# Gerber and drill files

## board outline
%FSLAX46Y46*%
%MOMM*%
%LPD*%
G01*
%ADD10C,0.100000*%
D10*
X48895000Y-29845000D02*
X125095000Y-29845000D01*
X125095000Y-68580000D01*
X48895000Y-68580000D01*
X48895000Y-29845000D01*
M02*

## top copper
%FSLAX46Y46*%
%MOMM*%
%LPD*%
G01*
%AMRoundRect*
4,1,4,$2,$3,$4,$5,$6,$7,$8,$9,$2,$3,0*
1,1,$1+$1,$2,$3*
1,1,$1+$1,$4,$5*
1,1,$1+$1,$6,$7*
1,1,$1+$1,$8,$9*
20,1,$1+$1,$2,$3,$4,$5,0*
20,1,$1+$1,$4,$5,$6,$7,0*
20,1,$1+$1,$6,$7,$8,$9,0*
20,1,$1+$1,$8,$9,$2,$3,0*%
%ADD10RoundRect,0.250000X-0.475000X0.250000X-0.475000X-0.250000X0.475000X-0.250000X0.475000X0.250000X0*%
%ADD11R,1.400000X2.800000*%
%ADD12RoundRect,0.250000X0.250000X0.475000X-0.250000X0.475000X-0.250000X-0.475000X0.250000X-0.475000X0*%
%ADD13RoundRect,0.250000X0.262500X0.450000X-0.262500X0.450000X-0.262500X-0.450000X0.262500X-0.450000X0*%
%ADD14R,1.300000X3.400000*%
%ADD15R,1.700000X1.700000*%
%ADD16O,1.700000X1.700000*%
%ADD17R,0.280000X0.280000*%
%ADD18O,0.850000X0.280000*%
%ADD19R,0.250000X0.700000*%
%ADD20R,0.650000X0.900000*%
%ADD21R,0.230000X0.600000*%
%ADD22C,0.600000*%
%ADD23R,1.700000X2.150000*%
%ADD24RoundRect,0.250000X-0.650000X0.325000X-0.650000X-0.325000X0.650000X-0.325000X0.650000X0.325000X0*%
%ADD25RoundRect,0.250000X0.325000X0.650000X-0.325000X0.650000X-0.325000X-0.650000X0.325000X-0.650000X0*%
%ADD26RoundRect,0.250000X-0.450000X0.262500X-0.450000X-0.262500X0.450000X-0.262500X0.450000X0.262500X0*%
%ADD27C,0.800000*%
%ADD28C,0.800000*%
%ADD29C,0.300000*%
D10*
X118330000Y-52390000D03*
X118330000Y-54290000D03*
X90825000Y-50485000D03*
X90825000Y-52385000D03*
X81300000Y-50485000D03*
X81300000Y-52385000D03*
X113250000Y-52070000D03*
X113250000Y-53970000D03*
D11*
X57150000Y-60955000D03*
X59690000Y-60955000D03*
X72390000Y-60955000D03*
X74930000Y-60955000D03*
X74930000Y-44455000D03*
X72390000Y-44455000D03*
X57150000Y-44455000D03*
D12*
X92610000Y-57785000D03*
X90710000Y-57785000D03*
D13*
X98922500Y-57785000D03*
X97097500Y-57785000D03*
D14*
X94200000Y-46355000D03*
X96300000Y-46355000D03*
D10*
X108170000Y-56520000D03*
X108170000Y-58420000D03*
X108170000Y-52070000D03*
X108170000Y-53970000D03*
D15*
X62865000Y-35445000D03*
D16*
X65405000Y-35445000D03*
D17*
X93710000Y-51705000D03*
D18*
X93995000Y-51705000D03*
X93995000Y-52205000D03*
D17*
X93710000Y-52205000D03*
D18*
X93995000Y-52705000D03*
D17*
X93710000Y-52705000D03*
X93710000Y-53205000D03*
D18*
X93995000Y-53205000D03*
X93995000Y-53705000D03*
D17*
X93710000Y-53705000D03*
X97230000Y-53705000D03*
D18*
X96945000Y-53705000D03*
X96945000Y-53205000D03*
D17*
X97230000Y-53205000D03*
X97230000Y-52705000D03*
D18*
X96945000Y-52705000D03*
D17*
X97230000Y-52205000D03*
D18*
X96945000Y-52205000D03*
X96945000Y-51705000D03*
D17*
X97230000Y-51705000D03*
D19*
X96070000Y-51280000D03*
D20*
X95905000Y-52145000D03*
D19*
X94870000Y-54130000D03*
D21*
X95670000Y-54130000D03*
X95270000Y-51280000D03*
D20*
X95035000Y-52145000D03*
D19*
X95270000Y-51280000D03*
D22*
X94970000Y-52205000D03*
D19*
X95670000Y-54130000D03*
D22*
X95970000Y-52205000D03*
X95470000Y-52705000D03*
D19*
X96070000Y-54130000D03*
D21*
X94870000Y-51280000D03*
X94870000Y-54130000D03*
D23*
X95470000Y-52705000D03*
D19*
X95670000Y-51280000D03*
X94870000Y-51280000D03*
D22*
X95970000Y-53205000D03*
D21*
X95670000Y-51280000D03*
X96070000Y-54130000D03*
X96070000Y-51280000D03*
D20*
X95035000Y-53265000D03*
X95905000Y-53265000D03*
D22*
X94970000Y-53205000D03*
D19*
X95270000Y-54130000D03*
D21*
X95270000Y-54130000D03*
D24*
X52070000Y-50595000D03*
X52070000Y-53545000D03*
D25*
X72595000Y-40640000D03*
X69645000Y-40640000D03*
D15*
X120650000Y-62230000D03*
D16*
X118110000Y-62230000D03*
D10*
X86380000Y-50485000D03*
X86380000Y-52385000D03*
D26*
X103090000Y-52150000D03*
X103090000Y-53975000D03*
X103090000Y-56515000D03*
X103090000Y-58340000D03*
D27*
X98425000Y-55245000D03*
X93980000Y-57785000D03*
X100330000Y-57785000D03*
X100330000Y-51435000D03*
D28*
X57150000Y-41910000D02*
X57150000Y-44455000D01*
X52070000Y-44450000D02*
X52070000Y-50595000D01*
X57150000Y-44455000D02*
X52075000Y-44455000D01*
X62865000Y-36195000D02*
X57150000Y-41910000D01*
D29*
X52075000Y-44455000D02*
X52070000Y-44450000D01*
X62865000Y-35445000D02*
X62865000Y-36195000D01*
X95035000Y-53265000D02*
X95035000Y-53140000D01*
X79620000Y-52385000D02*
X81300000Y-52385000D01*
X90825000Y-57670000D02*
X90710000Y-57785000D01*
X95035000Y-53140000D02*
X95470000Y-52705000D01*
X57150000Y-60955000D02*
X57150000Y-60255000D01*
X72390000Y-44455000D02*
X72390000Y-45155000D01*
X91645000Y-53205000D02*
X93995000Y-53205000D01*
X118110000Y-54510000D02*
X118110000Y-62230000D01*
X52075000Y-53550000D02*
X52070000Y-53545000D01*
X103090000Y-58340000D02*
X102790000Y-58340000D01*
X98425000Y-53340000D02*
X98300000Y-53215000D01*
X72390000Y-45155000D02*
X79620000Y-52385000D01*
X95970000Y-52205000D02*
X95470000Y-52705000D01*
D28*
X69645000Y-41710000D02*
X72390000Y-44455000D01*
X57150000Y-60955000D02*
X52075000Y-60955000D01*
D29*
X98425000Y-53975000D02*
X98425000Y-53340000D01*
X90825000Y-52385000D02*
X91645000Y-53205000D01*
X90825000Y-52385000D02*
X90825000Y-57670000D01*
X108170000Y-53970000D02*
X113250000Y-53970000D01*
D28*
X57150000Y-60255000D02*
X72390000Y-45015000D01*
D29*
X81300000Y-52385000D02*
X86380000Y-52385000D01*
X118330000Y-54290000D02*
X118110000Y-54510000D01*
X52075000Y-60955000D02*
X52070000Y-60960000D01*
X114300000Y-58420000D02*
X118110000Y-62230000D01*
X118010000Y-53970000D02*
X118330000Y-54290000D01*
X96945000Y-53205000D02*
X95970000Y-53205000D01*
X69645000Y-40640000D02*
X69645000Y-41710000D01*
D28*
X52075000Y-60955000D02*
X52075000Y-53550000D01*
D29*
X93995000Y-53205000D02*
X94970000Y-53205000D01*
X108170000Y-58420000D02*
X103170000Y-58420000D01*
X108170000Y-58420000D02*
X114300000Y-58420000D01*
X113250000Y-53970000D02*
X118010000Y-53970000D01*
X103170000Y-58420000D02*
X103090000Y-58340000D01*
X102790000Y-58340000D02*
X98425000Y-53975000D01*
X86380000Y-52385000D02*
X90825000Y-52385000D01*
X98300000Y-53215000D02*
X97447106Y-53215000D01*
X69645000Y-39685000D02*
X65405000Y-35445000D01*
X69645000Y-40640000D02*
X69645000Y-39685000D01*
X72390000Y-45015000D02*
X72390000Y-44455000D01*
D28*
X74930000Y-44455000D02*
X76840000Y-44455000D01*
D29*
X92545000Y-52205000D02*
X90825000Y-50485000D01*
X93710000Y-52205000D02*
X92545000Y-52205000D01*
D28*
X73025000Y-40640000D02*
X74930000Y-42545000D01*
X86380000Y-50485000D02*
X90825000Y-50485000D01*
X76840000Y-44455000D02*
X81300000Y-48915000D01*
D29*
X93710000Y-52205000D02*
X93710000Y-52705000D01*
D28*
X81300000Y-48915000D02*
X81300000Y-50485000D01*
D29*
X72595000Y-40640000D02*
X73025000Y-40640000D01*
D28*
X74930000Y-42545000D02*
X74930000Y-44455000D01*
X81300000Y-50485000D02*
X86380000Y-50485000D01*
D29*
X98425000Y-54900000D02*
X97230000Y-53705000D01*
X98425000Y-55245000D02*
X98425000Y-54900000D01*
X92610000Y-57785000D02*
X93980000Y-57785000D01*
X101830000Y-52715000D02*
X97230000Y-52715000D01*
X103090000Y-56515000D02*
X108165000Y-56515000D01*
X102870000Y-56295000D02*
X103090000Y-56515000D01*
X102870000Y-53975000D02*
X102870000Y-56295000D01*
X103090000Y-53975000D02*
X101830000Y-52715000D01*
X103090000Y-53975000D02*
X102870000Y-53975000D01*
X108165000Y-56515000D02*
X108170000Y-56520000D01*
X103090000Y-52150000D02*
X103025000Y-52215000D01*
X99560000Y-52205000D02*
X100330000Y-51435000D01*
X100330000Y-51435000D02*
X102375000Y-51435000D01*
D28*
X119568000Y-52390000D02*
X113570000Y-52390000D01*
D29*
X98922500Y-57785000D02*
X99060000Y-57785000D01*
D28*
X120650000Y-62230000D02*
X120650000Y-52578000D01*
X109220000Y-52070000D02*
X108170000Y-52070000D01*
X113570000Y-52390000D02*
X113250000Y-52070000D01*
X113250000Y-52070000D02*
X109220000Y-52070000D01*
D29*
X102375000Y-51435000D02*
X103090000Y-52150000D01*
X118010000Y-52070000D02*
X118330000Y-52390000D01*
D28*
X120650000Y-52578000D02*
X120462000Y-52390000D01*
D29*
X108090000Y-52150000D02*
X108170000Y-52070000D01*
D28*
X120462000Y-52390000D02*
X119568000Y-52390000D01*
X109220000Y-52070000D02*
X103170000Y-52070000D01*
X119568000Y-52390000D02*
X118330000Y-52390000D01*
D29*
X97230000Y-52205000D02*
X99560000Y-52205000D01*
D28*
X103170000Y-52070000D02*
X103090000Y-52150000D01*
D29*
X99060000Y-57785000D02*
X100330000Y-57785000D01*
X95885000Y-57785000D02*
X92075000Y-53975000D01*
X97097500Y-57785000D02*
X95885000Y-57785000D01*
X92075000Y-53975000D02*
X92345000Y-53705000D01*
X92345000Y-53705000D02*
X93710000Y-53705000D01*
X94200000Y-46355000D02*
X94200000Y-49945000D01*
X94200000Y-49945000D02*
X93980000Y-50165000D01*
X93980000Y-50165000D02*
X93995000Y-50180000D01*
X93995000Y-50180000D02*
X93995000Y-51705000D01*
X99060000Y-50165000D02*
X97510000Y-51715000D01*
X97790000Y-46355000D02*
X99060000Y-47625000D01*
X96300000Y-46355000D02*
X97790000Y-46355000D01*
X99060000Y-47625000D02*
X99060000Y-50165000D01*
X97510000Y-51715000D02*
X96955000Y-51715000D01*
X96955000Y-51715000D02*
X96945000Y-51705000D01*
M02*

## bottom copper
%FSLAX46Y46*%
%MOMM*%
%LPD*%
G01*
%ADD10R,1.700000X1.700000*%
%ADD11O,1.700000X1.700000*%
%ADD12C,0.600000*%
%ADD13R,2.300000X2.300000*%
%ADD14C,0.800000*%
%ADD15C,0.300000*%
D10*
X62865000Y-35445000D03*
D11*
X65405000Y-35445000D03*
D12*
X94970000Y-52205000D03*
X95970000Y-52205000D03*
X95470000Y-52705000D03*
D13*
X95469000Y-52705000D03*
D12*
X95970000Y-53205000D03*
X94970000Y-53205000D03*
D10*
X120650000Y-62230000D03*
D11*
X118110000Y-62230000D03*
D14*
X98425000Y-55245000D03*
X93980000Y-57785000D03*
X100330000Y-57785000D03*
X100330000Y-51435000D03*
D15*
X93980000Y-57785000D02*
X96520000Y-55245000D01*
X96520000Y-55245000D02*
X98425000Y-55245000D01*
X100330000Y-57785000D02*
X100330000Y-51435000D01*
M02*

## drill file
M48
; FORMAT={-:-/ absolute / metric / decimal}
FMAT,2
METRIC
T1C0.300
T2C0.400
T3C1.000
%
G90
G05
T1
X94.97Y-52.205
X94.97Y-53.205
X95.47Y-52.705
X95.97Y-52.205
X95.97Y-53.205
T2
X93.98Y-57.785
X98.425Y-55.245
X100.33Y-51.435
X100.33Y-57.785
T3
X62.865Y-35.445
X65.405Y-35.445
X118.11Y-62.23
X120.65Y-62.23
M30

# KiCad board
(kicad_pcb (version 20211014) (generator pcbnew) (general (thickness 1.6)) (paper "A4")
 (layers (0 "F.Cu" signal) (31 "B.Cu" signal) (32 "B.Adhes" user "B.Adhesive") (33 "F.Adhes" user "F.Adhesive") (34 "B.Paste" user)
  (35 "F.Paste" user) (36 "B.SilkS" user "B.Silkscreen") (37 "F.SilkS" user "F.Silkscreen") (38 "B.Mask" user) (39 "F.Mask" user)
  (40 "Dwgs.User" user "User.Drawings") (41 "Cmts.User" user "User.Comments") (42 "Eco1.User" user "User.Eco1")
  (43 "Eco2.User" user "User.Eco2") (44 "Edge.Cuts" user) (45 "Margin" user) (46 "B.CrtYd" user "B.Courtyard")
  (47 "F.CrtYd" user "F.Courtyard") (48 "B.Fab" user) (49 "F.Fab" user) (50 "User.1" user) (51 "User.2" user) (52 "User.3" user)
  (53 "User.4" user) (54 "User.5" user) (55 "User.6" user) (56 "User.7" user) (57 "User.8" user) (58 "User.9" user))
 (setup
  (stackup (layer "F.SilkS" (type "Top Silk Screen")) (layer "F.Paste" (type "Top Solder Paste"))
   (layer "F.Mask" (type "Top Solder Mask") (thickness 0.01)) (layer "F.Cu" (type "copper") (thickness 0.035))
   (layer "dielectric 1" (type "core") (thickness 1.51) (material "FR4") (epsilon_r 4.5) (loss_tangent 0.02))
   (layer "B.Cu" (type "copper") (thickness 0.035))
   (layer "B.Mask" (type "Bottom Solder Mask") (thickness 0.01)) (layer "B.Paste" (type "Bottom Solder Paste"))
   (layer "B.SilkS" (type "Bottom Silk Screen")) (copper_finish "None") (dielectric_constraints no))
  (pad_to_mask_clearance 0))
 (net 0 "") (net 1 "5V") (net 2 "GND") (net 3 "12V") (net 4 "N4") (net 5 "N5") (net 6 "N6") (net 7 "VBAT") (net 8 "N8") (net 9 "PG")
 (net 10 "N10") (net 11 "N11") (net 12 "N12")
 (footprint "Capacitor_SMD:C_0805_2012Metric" (layer "F.Cu") (at 118.33 53.34 -90)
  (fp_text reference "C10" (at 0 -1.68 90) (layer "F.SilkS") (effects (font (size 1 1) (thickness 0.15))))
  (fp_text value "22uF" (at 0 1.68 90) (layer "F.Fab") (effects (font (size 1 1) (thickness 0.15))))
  (pad "1" smd roundrect (at -0.95 0 270) (size 1 1.45) (layers "F.Cu" "F.Paste" "F.Mask") (roundrect_rratio 0.25) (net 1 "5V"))
  (pad "2" smd roundrect (at 0.95 0 270) (size 1 1.45) (layers "F.Cu" "F.Paste" "F.Mask") (roundrect_rratio 0.25) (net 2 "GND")))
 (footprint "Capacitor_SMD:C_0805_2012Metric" (layer "F.Cu") (at 90.825 51.435 -90)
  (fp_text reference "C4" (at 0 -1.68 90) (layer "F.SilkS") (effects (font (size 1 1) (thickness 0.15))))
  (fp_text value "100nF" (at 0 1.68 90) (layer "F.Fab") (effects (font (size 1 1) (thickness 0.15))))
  (pad "1" smd roundrect (at -0.95 0 270) (size 1 1.45) (layers "F.Cu" "F.Paste" "F.Mask") (roundrect_rratio 0.25) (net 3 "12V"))
  (pad "2" smd roundrect (at 0.95 0 270) (size 1 1.45) (layers "F.Cu" "F.Paste" "F.Mask") (roundrect_rratio 0.25) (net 2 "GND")))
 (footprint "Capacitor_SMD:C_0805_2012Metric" (layer "F.Cu") (at 81.3 51.435 -90)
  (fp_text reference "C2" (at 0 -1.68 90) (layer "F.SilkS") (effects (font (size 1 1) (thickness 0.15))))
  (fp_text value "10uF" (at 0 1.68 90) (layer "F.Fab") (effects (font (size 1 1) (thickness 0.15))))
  (pad "1" smd roundrect (at -0.95 0 270) (size 1 1.45) (layers "F.Cu" "F.Paste" "F.Mask") (roundrect_rratio 0.25) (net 3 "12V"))
  (pad "2" smd roundrect (at 0.95 0 270) (size 1 1.45) (layers "F.Cu" "F.Paste" "F.Mask") (roundrect_rratio 0.25) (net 2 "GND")))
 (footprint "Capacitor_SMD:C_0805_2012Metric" (layer "F.Cu") (at 113.25 53.02 -90)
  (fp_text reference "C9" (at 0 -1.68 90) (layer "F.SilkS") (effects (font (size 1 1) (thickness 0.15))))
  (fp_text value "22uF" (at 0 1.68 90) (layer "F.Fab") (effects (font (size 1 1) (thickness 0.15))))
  (pad "1" smd roundrect (at -0.95 0 270) (size 1 1.45) (layers "F.Cu" "F.Paste" "F.Mask") (roundrect_rratio 0.25) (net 1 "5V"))
  (pad "2" smd roundrect (at 0.95 0 270) (size 1 1.45) (layers "F.Cu" "F.Paste" "F.Mask") (roundrect_rratio 0.25) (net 2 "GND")))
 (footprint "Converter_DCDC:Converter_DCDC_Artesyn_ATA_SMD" (layer "F.Cu") (at 66.04 52.705 90)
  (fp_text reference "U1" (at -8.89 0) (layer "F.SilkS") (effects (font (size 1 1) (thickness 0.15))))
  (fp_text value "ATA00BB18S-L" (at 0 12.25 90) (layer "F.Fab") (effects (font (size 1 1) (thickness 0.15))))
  (pad "1" smd rect (at -8.25 -8.89 90) (size 2.8 1.4) (layers "F.Cu" "F.Paste" "F.Mask") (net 2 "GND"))
  (pad "2" smd rect (at -8.25 -6.35 90) (size 2.8 1.4) (layers "F.Cu" "F.Paste" "F.Mask") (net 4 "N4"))
  (pad "7" smd rect (at -8.25 6.35 90) (size 2.8 1.4) (layers "F.Cu" "F.Paste" "F.Mask") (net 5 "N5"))
  (pad "8" smd rect (at -8.25 8.89 90) (size 2.8 1.4) (layers "F.Cu" "F.Paste" "F.Mask") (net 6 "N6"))
  (pad "9" smd rect (at 8.25 8.89 90) (size 2.8 1.4) (layers "F.Cu" "F.Paste" "F.Mask") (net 3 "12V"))
  (pad "10" smd rect (at 8.25 6.35 90) (size 2.8 1.4) (layers "F.Cu" "F.Paste" "F.Mask") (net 2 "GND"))
  (pad "16" smd rect (at 8.25 -8.89 90) (size 2.8 1.4) (layers "F.Cu" "F.Paste" "F.Mask") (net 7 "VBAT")))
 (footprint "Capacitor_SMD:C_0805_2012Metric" (layer "F.Cu") (at 91.66 57.785 180)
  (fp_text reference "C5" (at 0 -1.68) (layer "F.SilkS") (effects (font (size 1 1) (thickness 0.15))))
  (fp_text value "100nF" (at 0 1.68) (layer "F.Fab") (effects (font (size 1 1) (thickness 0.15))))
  (pad "1" smd roundrect (at -0.95 0 180) (size 1 1.45) (layers "F.Cu" "F.Paste" "F.Mask") (roundrect_rratio 0.25) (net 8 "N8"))
  (pad "2" smd roundrect (at 0.95 0 180) (size 1 1.45) (layers "F.Cu" "F.Paste" "F.Mask") (roundrect_rratio 0.25) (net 2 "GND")))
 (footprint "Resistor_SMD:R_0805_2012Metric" (layer "F.Cu") (at 98.01 57.785 180)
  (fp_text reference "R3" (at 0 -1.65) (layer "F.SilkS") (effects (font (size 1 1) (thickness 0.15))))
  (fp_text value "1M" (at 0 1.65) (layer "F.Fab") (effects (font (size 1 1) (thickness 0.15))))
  (pad "1" smd roundrect (at -0.9125 0 180) (size 1.025 1.4) (layers "F.Cu" "F.Paste" "F.Mask") (roundrect_rratio 0.243902439) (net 1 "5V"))
  (pad "2" smd roundrect (at 0.9125 0 180) (size 1.025 1.4) (layers "F.Cu" "F.Paste" "F.Mask") (roundrect_rratio 0.243902439) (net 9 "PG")))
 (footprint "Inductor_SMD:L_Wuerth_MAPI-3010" (layer "F.Cu") (at 95.25 46.355)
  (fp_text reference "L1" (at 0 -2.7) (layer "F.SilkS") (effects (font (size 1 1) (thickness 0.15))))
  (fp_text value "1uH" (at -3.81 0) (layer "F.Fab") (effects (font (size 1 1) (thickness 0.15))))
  (pad "1" smd rect (at -1.05 0) (size 1.3 3.4) (layers "F.Cu" "F.Paste" "F.Mask") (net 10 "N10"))
  (pad "2" smd rect (at 1.05 0) (size 1.3 3.4) (layers "F.Cu" "F.Paste" "F.Mask") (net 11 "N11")))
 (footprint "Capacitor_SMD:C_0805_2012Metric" (layer "F.Cu") (at 108.17 57.47 -90)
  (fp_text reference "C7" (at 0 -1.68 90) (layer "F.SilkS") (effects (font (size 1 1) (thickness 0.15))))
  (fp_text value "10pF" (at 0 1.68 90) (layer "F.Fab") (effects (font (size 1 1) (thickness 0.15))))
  (pad "1" smd roundrect (at -0.95 0 270) (size 1 1.45) (layers "F.Cu" "F.Paste" "F.Mask") (roundrect_rratio 0.25) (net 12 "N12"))
  (pad "2" smd roundrect (at 0.95 0 270) (size 1 1.45) (layers "F.Cu" "F.Paste" "F.Mask") (roundrect_rratio 0.25) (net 2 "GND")))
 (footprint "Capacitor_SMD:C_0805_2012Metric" (layer "F.Cu") (at 108.17 53.02 -90)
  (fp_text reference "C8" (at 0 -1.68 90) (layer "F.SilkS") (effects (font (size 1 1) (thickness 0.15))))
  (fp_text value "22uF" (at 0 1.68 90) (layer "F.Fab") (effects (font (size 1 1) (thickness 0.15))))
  (pad "1" smd roundrect (at -0.95 0 270) (size 1 1.45) (layers "F.Cu" "F.Paste" "F.Mask") (roundrect_rratio 0.25) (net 1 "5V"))
  (pad "2" smd roundrect (at 0.95 0 270) (size 1 1.45) (layers "F.Cu" "F.Paste" "F.Mask") (roundrect_rratio 0.25) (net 2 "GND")))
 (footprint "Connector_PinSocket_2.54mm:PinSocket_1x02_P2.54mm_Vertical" (layer "F.Cu") (at 62.865 35.445 90)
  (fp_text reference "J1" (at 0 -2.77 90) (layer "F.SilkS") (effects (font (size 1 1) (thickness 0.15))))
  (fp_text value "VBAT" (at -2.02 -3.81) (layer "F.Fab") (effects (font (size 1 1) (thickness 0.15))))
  (pad "1" thru_hole rect (at 0 0 90) (size 1.7 1.7) (drill 1) (layers *.Cu *.Mask) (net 7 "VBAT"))
  (pad "2" thru_hole oval (at 0 2.54 90) (size 1.7 1.7) (drill 1) (layers *.Cu *.Mask) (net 2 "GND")))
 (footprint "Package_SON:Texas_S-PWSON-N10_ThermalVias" (layer "F.Cu") (at 95.47 52.705)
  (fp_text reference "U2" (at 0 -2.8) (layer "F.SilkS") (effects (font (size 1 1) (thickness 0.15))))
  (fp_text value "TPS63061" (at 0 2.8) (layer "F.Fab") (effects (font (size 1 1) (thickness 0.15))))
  (pad "1" smd rect (at -1.76 -1) (size 0.28 0.28) (layers "F.Cu" "F.Paste" "F.Mask") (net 10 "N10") (solder_mask_margin 0.07)
   (solder_paste_margin -0.025))
  (pad "1" smd oval (at -1.475 -1) (size 0.85 0.28) (layers "F.Cu" "F.Paste" "F.Mask") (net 10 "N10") (solder_mask_margin 0.07)
   (solder_paste_margin -0.025))
  (pad "2" smd oval (at -1.475 -0.5) (size 0.85 0.28) (layers "F.Cu" "F.Paste" "F.Mask") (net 3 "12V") (solder_mask_margin 0.07)
   (solder_paste_margin -0.025))
  (pad "2" smd rect (at -1.76 -0.5) (size 0.28 0.28) (layers "F.Cu" "F.Paste" "F.Mask") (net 3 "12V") (solder_mask_margin 0.07)
   (solder_paste_margin -0.025))
  (pad "3" smd oval (at -1.475 0) (size 0.85 0.28) (layers "F.Cu" "F.Paste" "F.Mask") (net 3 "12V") (solder_mask_margin 0.07)
   (solder_paste_margin -0.025))
  (pad "3" smd rect (at -1.76 0) (size 0.28 0.28) (layers "F.Cu" "F.Paste" "F.Mask") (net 3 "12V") (solder_mask_margin 0.07)
   (solder_paste_margin -0.025))
  (pad "4" smd rect (at -1.76 0.5) (size 0.28 0.28) (layers "F.Cu" "F.Paste" "F.Mask") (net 2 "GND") (solder_mask_margin 0.07)
   (solder_paste_margin -0.025))
  (pad "4" smd oval (at -1.475 0.5) (size 0.85 0.28) (layers "F.Cu" "F.Paste" "F.Mask") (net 2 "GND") (solder_mask_margin 0.07)
   (solder_paste_margin -0.025))
  (pad "5" smd oval (at -1.475 1) (size 0.85 0.28) (layers "F.Cu" "F.Paste" "F.Mask") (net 9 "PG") (solder_mask_margin 0.07)
   (solder_paste_margin -0.025))
  (pad "5" smd rect (at -1.76 1) (size 0.28 0.28) (layers "F.Cu" "F.Paste" "F.Mask") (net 9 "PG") (solder_mask_margin 0.07)
   (solder_paste_margin -0.025))
  (pad "6" smd rect (at 1.76 1) (size 0.28 0.28) (layers "F.Cu" "F.Paste" "F.Mask") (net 8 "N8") (solder_mask_margin 0.07)
   (solder_paste_margin -0.025))
  (pad "6" smd oval (at 1.475 1) (size 0.85 0.28) (layers "F.Cu" "F.Paste" "F.Mask") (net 8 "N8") (solder_mask_margin 0.07)
   (solder_paste_margin -0.025))
  (pad "7" smd oval (at 1.475 0.5) (size 0.85 0.28) (layers "F.Cu" "F.Paste" "F.Mask") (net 2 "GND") (solder_mask_margin 0.07)
   (solder_paste_margin -0.025))
  (pad "7" smd rect (at 1.76 0.5) (size 0.28 0.28) (layers "F.Cu" "F.Paste" "F.Mask") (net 2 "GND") (solder_mask_margin 0.07)
   (solder_paste_margin -0.025))
  (pad "8" smd rect (at 1.76 0) (size 0.28 0.28) (layers "F.Cu" "F.Paste" "F.Mask") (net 12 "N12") (solder_mask_margin 0.07)
   (solder_paste_margin -0.025))
  (pad "8" smd oval (at 1.475 0) (size 0.85 0.28) (layers "F.Cu" "F.Paste" "F.Mask") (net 12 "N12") (solder_mask_margin 0.07)
   (solder_paste_margin -0.025))
  (pad "9" smd rect (at 1.76 -0.5) (size 0.28 0.28) (layers "F.Cu" "F.Paste" "F.Mask") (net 1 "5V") (solder_mask_margin 0.07)
   (solder_paste_margin -0.025))
  (pad "9" smd oval (at 1.475 -0.5) (size 0.85 0.28) (layers "F.Cu" "F.Paste" "F.Mask") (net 1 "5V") (solder_mask_margin 0.07)
   (solder_paste_margin -0.025))
  (pad "10" smd oval (at 1.475 -1) (size 0.85 0.28) (layers "F.Cu" "F.Paste" "F.Mask") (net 11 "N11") (solder_mask_margin 0.07)
   (solder_paste_margin -0.025))
  (pad "10" smd rect (at 1.76 -1) (size 0.28 0.28) (layers "F.Cu" "F.Paste" "F.Mask") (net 11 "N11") (solder_mask_margin 0.07)
   (solder_paste_margin -0.025))
  (pad "11" smd rect (at 0.6 -1.425) (size 0.25 0.7) (layers "F.Cu" "F.Paste" "F.Mask") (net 2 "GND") (solder_paste_margin -0.05))
  (pad "11" smd rect (at 0.435 -0.56) (size 0.65 0.9) (layers "F.Cu" "F.Paste" "F.Mask") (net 2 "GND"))
  (pad "11" smd rect (at -0.6 1.425) (size 0.25 0.7) (layers "F.Cu" "F.Paste" "F.Mask") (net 2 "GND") (solder_paste_margin -0.05))
  (pad "11" smd rect (at 0.2 1.425) (size 0.23 0.6) (layers "F.Cu" "F.Paste" "F.Mask") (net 2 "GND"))
  (pad "11" smd rect (at -0.2 -1.425) (size 0.23 0.6) (layers "F.Cu" "F.Paste" "F.Mask") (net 2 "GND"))
  (pad "11" smd rect (at -0.435 -0.56) (size 0.65 0.9) (layers "F.Cu" "F.Paste" "F.Mask") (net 2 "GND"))
  (pad "11" smd rect (at -0.2 -1.425) (size 0.25 0.7) (layers "F.Cu" "F.Paste" "F.Mask") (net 2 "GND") (solder_paste_margin -0.05))
  (pad "11" thru_hole circle (at -0.5 -0.5) (size 0.6 0.6) (drill 0.3) (layers *.Cu *.Mask) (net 2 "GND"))
  (pad "11" smd rect (at 0.2 1.425) (size 0.25 0.7) (layers "F.Cu" "F.Paste" "F.Mask") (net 2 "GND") (solder_paste_margin -0.05))
  (pad "11" thru_hole circle (at 0.5 -0.5) (size 0.6 0.6) (drill 0.3) (layers *.Cu *.Mask) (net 2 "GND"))
  (pad "11" thru_hole circle (at 0 0) (size 0.6 0.6) (drill 0.3) (layers *.Cu *.Mask) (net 2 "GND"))
  (pad "11" smd rect (at 0.6 1.425) (size 0.25 0.7) (layers "F.Cu" "F.Paste" "F.Mask") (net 2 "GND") (solder_paste_margin -0.05))
  (pad "11" smd rect (at -0.6 -1.425) (size 0.23 0.6) (layers "F.Cu" "F.Paste" "F.Mask") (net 2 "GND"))
  (pad "11" smd rect (at -0.6 1.425) (size 0.23 0.6) (layers "F.Cu" "F.Paste" "F.Mask") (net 2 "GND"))
  (pad "11" smd rect (at 0 0) (size 1.7 2.15) (layers "F.Cu" "F.Mask") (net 2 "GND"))
  (pad "11" smd rect (at -0.001 0) (size 2.3 2.3) (layers "B.Cu") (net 2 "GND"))
  (pad "11" smd rect (at 0.2 -1.425) (size 0.25 0.7) (layers "F.Cu" "F.Paste" "F.Mask") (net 2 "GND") (solder_paste_margin -0.05))
  (pad "11" smd rect (at -0.6 -1.425) (size 0.25 0.7) (layers "F.Cu" "F.Paste" "F.Mask") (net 2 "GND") (solder_paste_margin -0.05))
  (pad "11" thru_hole circle (at 0.5 0.5) (size 0.6 0.6) (drill 0.3) (layers *.Cu *.Mask) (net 2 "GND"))
  (pad "11" smd rect (at 0.2 -1.425) (size 0.23 0.6) (layers "F.Cu" "F.Paste" "F.Mask") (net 2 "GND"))
  (pad "11" smd rect (at 0.6 1.425) (size 0.23 0.6) (layers "F.Cu" "F.Paste" "F.Mask") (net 2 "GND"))
  (pad "11" smd rect (at 0.6 -1.425) (size 0.23 0.6) (layers "F.Cu" "F.Paste" "F.Mask") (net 2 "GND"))
  (pad "11" smd rect (at -0.435 0.56) (size 0.65 0.9) (layers "F.Cu" "F.Paste" "F.Mask") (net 2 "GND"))
  (pad "11" smd rect (at 0.435 0.56) (size 0.65 0.9) (layers "F.Cu" "F.Paste" "F.Mask") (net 2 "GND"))
  (pad "11" thru_hole circle (at -0.5 0.5) (size 0.6 0.6) (drill 0.3) (layers *.Cu *.Mask) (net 2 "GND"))
  (pad "11" smd rect (at -0.2 1.425) (size 0.25 0.7) (layers "F.Cu" "F.Paste" "F.Mask") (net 2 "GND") (solder_paste_margin -0.05))
  (pad "11" smd rect (at -0.2 1.425) (size 0.23 0.6) (layers "F.Cu" "F.Paste" "F.Mask") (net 2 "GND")))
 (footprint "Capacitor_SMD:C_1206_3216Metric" (layer "F.Cu") (at 52.07 52.07 -90)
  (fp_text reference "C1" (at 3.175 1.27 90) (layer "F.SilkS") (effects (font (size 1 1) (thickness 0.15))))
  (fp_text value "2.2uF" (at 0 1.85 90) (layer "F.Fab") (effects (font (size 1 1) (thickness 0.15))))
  (pad "1" smd roundrect (at -1.475 0 270) (size 1.15 1.8) (layers "F.Cu" "F.Paste" "F.Mask") (roundrect_rratio 0.2173913043) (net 7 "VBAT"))
  (pad "2" smd roundrect (at 1.475 0 270) (size 1.15 1.8) (layers "F.Cu" "F.Paste" "F.Mask") (roundrect_rratio 0.2173913043) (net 2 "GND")))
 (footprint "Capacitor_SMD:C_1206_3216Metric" (layer "F.Cu") (at 71.12 40.64 180)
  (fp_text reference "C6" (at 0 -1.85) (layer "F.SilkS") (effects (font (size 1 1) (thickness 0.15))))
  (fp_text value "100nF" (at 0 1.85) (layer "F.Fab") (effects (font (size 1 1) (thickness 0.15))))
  (pad "1" smd roundrect (at -1.475 0 180) (size 1.15 1.8) (layers "F.Cu" "F.Paste" "F.Mask") (roundrect_rratio 0.2173913043) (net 3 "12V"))
  (pad "2" smd roundrect (at 1.475 0 180) (size 1.15 1.8) (layers "F.Cu" "F.Paste" "F.Mask") (roundrect_rratio 0.2173913043) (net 2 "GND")))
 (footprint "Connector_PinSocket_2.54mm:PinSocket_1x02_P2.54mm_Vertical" (layer "F.Cu") (at 120.65 62.23 -90)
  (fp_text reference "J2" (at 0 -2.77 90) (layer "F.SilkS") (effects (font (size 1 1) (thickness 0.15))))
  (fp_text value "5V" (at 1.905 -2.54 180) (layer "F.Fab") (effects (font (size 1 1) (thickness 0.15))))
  (pad "1" thru_hole rect (at 0 0 270) (size 1.7 1.7) (drill 1) (layers *.Cu *.Mask) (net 1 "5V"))
  (pad "2" thru_hole oval (at 0 2.54 270) (size 1.7 1.7) (drill 1) (layers *.Cu *.Mask) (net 2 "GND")))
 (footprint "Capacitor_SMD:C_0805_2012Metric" (layer "F.Cu") (at 86.38 51.435 -90)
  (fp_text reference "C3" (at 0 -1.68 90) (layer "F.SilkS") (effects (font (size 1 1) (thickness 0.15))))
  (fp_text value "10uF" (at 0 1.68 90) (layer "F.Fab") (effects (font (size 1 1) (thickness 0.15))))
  (pad "1" smd roundrect (at -0.95 0 270) (size 1 1.45) (layers "F.Cu" "F.Paste" "F.Mask") (roundrect_rratio 0.25) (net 3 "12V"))
  (pad "2" smd roundrect (at 0.95 0 270) (size 1 1.45) (layers "F.Cu" "F.Paste" "F.Mask") (roundrect_rratio 0.25) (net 2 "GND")))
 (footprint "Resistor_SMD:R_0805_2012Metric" (layer "F.Cu") (at 103.09 53.0625 -90)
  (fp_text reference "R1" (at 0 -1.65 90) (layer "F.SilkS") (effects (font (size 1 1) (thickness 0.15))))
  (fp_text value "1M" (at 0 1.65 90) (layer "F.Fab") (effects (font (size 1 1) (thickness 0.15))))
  (pad "1" smd roundrect (at -0.9125 0 270) (size 1.025 1.4) (layers "F.Cu" "F.Paste" "F.Mask") (roundrect_rratio 0.243902439) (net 1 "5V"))
  (pad "2" smd roundrect (at 0.9125 0 270) (size 1.025 1.4) (layers "F.Cu" "F.Paste" "F.Mask") (roundrect_rratio 0.243902439) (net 12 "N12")))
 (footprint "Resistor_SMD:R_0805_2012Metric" (layer "F.Cu") (at 103.09 57.4275 -90)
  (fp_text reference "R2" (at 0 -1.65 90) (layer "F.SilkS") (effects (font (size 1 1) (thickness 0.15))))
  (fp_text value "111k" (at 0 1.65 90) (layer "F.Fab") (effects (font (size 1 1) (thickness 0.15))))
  (pad "1" smd roundrect (at -0.9125 0 270) (size 1.025 1.4) (layers "F.Cu" "F.Paste" "F.Mask") (roundrect_rratio 0.243902439)
   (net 12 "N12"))
  (pad "2" smd roundrect (at 0.9125 0 270) (size 1.025 1.4) (layers "F.Cu" "F.Paste" "F.Mask") (roundrect_rratio 0.243902439) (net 2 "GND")))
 (gr_rect (start 48.895 29.845) (end 125.095 68.58) (layer "Edge.Cuts") (width 0.1) (fill none))
 (segment (start 57.15 41.91) (end 57.15 44.455) (width 0.8) (layer "F.Cu") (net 7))
 (segment (start 52.07 44.45) (end 52.07 50.595) (width 0.8) (layer "F.Cu") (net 7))
 (segment (start 57.15 44.455) (end 52.075 44.455) (width 0.8) (layer "F.Cu") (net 7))
 (segment (start 62.865 36.195) (end 57.15 41.91) (width 0.8) (layer "F.Cu") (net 7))
 (segment (start 52.075 44.455) (end 52.07 44.45) (width 0.3) (layer "F.Cu") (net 7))
 (segment (start 62.865 35.445) (end 62.865 36.195) (width 0.3) (layer "F.Cu") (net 7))
 (segment (start 95.035 53.265) (end 95.035 53.14) (width 0.3) (layer "F.Cu") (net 2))
 (segment (start 79.62 52.385) (end 81.3 52.385) (width 0.3) (layer "F.Cu") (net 2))
 (segment (start 90.825 57.67) (end 90.71 57.785) (width 0.3) (layer "F.Cu") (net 2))
 (segment (start 95.035 53.14) (end 95.47 52.705) (width 0.3) (layer "F.Cu") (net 2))
 (segment (start 57.15 60.955) (end 57.15 60.255) (width 0.3) (layer "F.Cu") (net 2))
 (segment (start 72.39 44.455) (end 72.39 45.155) (width 0.3) (layer "F.Cu") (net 2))
 (segment (start 91.645 53.205) (end 93.995 53.205) (width 0.3) (layer "F.Cu") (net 2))
 (segment (start 118.11 54.51) (end 118.11 62.23) (width 0.3) (layer "F.Cu") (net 2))
 (segment (start 52.075 53.55) (end 52.07 53.545) (width 0.3) (layer "F.Cu") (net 2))
 (segment (start 103.09 58.34) (end 102.79 58.34) (width 0.3) (layer "F.Cu") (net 2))
 (segment (start 98.425 53.34) (end 98.3 53.215) (width 0.3) (layer "F.Cu") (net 2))
 (segment (start 72.39 45.155) (end 79.62 52.385) (width 0.3) (layer "F.Cu") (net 2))
 (segment (start 95.97 52.205) (end 95.47 52.705) (width 0.3) (layer "F.Cu") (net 2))
 (segment (start 69.645 41.71) (end 72.39 44.455) (width 0.8) (layer "F.Cu") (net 2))
 (segment (start 57.15 60.955) (end 52.075 60.955) (width 0.8) (layer "F.Cu") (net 2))
 (segment (start 98.425 53.975) (end 98.425 53.34) (width 0.3) (layer "F.Cu") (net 2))
 (segment (start 90.825 52.385) (end 91.645 53.205) (width 0.3) (layer "F.Cu") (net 2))
 (segment (start 90.825 52.385) (end 90.825 57.67) (width 0.3) (layer "F.Cu") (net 2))
 (segment (start 108.17 53.97) (end 113.25 53.97) (width 0.3) (layer "F.Cu") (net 2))
 (segment (start 57.15 60.255) (end 72.39 45.015) (width 0.8) (layer "F.Cu") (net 2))
 (segment (start 81.3 52.385) (end 86.38 52.385) (width 0.3) (layer "F.Cu") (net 2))
 (segment (start 118.33 54.29) (end 118.11 54.51) (width 0.3) (layer "F.Cu") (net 2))
 (segment (start 52.075 60.955) (end 52.07 60.96) (width 0.3) (layer "F.Cu") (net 2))
 (segment (start 114.3 58.42) (end 118.11 62.23) (width 0.3) (layer "F.Cu") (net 2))
 (segment (start 118.01 53.97) (end 118.33 54.29) (width 0.3) (layer "F.Cu") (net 2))
 (segment (start 96.945 53.205) (end 95.97 53.205) (width 0.3) (layer "F.Cu") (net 2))
 (segment (start 69.645 40.64) (end 69.645 41.71) (width 0.3) (layer "F.Cu") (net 2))
 (segment (start 52.075 60.955) (end 52.075 53.55) (width 0.8) (layer "F.Cu") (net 2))
 (segment (start 93.995 53.205) (end 94.97 53.205) (width 0.3) (layer "F.Cu") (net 2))
 (segment (start 108.17 58.42) (end 103.17 58.42) (width 0.3) (layer "F.Cu") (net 2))
 (segment (start 108.17 58.42) (end 114.3 58.42) (width 0.3) (layer "F.Cu") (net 2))
 (segment (start 113.25 53.97) (end 118.01 53.97) (width 0.3) (layer "F.Cu") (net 2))
 (segment (start 103.17 58.42) (end 103.09 58.34) (width 0.3) (layer "F.Cu") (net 2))
 (segment (start 102.79 58.34) (end 98.425 53.975) (width 0.3) (layer "F.Cu") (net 2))
 (segment (start 86.38 52.385) (end 90.825 52.385) (width 0.3) (layer "F.Cu") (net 2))
 (segment (start 98.3 53.215) (end 97.447106 53.215) (width 0.3) (layer "F.Cu") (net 2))
 (segment (start 69.645 39.685) (end 65.405 35.445) (width 0.3) (layer "F.Cu") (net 2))
 (segment (start 69.645 40.64) (end 69.645 39.685) (width 0.3) (layer "F.Cu") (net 2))
 (segment (start 72.39 45.015) (end 72.39 44.455) (width 0.3) (layer "F.Cu") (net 2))
 (segment (start 74.93 44.455) (end 76.84 44.455) (width 0.8) (layer "F.Cu") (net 3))
 (segment (start 92.545 52.205) (end 90.825 50.485) (width 0.3) (layer "F.Cu") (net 3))
 (segment (start 93.71 52.205) (end 92.545 52.205) (width 0.3) (layer "F.Cu") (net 3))
 (segment (start 73.025 40.64) (end 74.93 42.545) (width 0.8) (layer "F.Cu") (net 3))
 (segment (start 86.38 50.485) (end 90.825 50.485) (width 0.8) (layer "F.Cu") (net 3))
 (segment (start 76.84 44.455) (end 81.3 48.915) (width 0.8) (layer "F.Cu") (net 3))
 (segment (start 93.71 52.205) (end 93.71 52.705) (width 0.3) (layer "F.Cu") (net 3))
 (segment (start 81.3 48.915) (end 81.3 50.485) (width 0.8) (layer "F.Cu") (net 3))
 (segment (start 72.595 40.64) (end 73.025 40.64) (width 0.3) (layer "F.Cu") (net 3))
 (segment (start 74.93 42.545) (end 74.93 44.455) (width 0.8) (layer "F.Cu") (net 3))
 (segment (start 81.3 50.485) (end 86.38 50.485) (width 0.8) (layer "F.Cu") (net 3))
 (segment (start 98.425 54.9) (end 97.23 53.705) (width 0.3) (layer "F.Cu") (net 8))
 (segment (start 98.425 55.245) (end 98.425 54.9) (width 0.3) (layer "F.Cu") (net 8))
 (segment (start 92.61 57.785) (end 93.98 57.785) (width 0.3) (layer "F.Cu") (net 8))
 (via (at 98.425 55.245) (size 0.8) (drill 0.4) (layers "F.Cu" "B.Cu") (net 8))
 (via (at 93.98 57.785) (size 0.8) (drill 0.4) (layers "F.Cu" "B.Cu") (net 8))
 (segment (start 93.98 57.785) (end 96.52 55.245) (width 0.3) (layer "B.Cu") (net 8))
 (segment (start 96.52 55.245) (end 98.425 55.245) (width 0.3) (layer "B.Cu") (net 8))
 (segment (start 101.83 52.715) (end 97.23 52.715) (width 0.3) (layer "F.Cu") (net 12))
 (segment (start 103.09 56.515) (end 108.165 56.515) (width 0.3) (layer "F.Cu") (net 12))
 (segment (start 102.87 56.295) (end 103.09 56.515) (width 0.3) (layer "F.Cu") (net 12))
 (segment (start 102.87 53.975) (end 102.87 56.295) (width 0.3) (layer "F.Cu") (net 12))
 (segment (start 103.09 53.975) (end 101.83 52.715) (width 0.3) (layer "F.Cu") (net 12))
 (segment (start 103.09 53.975) (end 102.87 53.975) (width 0.3) (layer "F.Cu") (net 12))
 (segment (start 108.165 56.515) (end 108.17 56.52) (width 0.3) (layer "F.Cu") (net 12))
 (segment (start 103.09 52.15) (end 103.025 52.215) (width 0.3) (layer "F.Cu") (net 1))
 (segment (start 99.56 52.205) (end 100.33 51.435) (width 0.3) (layer "F.Cu") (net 1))
 (segment (start 100.33 51.435) (end 102.375 51.435) (width 0.3) (layer "F.Cu") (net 1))
 (segment (start 119.568 52.39) (end 113.57 52.39) (width 0.8) (layer "F.Cu") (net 1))
 (segment (start 98.9225 57.785) (end 99.06 57.785) (width 0.3) (layer "F.Cu") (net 1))
 (segment (start 120.65 62.23) (end 120.65 52.578) (width 0.8) (layer "F.Cu") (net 1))
 (segment (start 109.22 52.07) (end 108.17 52.07) (width 0.8) (layer "F.Cu") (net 1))
 (segment (start 113.57 52.39) (end 113.25 52.07) (width 0.8) (layer "F.Cu") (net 1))
 (segment (start 113.25 52.07) (end 109.22 52.07) (width 0.8) (layer "F.Cu") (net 1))
 (segment (start 102.375 51.435) (end 103.09 52.15) (width 0.3) (layer "F.Cu") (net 1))
 (segment (start 118.01 52.07) (end 118.33 52.39) (width 0.3) (layer "F.Cu") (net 1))
 (segment (start 120.65 52.578) (end 120.462 52.39) (width 0.8) (layer "F.Cu") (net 1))
 (segment (start 108.09 52.15) (end 108.17 52.07) (width 0.3) (layer "F.Cu") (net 1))
 (segment (start 120.462 52.39) (end 119.568 52.39) (width 0.8) (layer "F.Cu") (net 1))
 (segment (start 109.22 52.07) (end 103.17 52.07) (width 0.8) (layer "F.Cu") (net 1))
 (segment (start 119.568 52.39) (end 118.33 52.39) (width 0.8) (layer "F.Cu") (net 1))
 (segment (start 97.23 52.205) (end 99.56 52.205) (width 0.3) (layer "F.Cu") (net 1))
 (segment (start 103.17 52.07) (end 103.09 52.15) (width 0.8) (layer "F.Cu") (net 1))
 (segment (start 99.06 57.785) (end 100.33 57.785) (width 0.3) (layer "F.Cu") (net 1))
 (via (at 100.33 57.785) (size 0.8) (drill 0.4) (layers "F.Cu" "B.Cu") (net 1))
 (via (at 100.33 51.435) (size 0.8) (drill 0.4) (layers "F.Cu" "B.Cu") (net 1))
 (segment (start 100.33 57.785) (end 100.33 51.435) (width 0.3) (layer "B.Cu") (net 1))
 (segment (start 95.885 57.785) (end 92.075 53.975) (width 0.3) (layer "F.Cu") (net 9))
 (segment (start 97.0975 57.785) (end 95.885 57.785) (width 0.3) (layer "F.Cu") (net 9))
 (segment (start 92.075 53.975) (end 92.345 53.705) (width 0.3) (layer "F.Cu") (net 9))
 (segment (start 92.345 53.705) (end 93.71 53.705) (width 0.3) (layer "F.Cu") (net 9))
 (segment (start 94.2 46.355) (end 94.2 49.945) (width 0.3) (layer "F.Cu") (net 10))
 (segment (start 94.2 49.945) (end 93.98 50.165) (width 0.3) (layer "F.Cu") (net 10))
 (segment (start 93.98 50.165) (end 93.995 50.18) (width 0.3) (layer "F.Cu") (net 10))
 (segment (start 93.995 50.18) (end 93.995 51.705) (width 0.3) (layer "F.Cu") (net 10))
 (segment (start 99.06 50.165) (end 97.51 51.715) (width 0.3) (layer "F.Cu") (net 11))
 (segment (start 97.79 46.355) (end 99.06 47.625) (width 0.3) (layer "F.Cu") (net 11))
 (segment (start 96.3 46.355) (end 97.79 46.355) (width 0.3) (layer "F.Cu") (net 11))
 (segment (start 99.06 47.625) (end 99.06 50.165) (width 0.3) (layer "F.Cu") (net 11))
 (segment (start 97.51 51.715) (end 96.955 51.715) (width 0.3) (layer "F.Cu") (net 11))
 (segment (start 96.955 51.715) (end 96.945 51.705) (width 0.3) (layer "F.Cu") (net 11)))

